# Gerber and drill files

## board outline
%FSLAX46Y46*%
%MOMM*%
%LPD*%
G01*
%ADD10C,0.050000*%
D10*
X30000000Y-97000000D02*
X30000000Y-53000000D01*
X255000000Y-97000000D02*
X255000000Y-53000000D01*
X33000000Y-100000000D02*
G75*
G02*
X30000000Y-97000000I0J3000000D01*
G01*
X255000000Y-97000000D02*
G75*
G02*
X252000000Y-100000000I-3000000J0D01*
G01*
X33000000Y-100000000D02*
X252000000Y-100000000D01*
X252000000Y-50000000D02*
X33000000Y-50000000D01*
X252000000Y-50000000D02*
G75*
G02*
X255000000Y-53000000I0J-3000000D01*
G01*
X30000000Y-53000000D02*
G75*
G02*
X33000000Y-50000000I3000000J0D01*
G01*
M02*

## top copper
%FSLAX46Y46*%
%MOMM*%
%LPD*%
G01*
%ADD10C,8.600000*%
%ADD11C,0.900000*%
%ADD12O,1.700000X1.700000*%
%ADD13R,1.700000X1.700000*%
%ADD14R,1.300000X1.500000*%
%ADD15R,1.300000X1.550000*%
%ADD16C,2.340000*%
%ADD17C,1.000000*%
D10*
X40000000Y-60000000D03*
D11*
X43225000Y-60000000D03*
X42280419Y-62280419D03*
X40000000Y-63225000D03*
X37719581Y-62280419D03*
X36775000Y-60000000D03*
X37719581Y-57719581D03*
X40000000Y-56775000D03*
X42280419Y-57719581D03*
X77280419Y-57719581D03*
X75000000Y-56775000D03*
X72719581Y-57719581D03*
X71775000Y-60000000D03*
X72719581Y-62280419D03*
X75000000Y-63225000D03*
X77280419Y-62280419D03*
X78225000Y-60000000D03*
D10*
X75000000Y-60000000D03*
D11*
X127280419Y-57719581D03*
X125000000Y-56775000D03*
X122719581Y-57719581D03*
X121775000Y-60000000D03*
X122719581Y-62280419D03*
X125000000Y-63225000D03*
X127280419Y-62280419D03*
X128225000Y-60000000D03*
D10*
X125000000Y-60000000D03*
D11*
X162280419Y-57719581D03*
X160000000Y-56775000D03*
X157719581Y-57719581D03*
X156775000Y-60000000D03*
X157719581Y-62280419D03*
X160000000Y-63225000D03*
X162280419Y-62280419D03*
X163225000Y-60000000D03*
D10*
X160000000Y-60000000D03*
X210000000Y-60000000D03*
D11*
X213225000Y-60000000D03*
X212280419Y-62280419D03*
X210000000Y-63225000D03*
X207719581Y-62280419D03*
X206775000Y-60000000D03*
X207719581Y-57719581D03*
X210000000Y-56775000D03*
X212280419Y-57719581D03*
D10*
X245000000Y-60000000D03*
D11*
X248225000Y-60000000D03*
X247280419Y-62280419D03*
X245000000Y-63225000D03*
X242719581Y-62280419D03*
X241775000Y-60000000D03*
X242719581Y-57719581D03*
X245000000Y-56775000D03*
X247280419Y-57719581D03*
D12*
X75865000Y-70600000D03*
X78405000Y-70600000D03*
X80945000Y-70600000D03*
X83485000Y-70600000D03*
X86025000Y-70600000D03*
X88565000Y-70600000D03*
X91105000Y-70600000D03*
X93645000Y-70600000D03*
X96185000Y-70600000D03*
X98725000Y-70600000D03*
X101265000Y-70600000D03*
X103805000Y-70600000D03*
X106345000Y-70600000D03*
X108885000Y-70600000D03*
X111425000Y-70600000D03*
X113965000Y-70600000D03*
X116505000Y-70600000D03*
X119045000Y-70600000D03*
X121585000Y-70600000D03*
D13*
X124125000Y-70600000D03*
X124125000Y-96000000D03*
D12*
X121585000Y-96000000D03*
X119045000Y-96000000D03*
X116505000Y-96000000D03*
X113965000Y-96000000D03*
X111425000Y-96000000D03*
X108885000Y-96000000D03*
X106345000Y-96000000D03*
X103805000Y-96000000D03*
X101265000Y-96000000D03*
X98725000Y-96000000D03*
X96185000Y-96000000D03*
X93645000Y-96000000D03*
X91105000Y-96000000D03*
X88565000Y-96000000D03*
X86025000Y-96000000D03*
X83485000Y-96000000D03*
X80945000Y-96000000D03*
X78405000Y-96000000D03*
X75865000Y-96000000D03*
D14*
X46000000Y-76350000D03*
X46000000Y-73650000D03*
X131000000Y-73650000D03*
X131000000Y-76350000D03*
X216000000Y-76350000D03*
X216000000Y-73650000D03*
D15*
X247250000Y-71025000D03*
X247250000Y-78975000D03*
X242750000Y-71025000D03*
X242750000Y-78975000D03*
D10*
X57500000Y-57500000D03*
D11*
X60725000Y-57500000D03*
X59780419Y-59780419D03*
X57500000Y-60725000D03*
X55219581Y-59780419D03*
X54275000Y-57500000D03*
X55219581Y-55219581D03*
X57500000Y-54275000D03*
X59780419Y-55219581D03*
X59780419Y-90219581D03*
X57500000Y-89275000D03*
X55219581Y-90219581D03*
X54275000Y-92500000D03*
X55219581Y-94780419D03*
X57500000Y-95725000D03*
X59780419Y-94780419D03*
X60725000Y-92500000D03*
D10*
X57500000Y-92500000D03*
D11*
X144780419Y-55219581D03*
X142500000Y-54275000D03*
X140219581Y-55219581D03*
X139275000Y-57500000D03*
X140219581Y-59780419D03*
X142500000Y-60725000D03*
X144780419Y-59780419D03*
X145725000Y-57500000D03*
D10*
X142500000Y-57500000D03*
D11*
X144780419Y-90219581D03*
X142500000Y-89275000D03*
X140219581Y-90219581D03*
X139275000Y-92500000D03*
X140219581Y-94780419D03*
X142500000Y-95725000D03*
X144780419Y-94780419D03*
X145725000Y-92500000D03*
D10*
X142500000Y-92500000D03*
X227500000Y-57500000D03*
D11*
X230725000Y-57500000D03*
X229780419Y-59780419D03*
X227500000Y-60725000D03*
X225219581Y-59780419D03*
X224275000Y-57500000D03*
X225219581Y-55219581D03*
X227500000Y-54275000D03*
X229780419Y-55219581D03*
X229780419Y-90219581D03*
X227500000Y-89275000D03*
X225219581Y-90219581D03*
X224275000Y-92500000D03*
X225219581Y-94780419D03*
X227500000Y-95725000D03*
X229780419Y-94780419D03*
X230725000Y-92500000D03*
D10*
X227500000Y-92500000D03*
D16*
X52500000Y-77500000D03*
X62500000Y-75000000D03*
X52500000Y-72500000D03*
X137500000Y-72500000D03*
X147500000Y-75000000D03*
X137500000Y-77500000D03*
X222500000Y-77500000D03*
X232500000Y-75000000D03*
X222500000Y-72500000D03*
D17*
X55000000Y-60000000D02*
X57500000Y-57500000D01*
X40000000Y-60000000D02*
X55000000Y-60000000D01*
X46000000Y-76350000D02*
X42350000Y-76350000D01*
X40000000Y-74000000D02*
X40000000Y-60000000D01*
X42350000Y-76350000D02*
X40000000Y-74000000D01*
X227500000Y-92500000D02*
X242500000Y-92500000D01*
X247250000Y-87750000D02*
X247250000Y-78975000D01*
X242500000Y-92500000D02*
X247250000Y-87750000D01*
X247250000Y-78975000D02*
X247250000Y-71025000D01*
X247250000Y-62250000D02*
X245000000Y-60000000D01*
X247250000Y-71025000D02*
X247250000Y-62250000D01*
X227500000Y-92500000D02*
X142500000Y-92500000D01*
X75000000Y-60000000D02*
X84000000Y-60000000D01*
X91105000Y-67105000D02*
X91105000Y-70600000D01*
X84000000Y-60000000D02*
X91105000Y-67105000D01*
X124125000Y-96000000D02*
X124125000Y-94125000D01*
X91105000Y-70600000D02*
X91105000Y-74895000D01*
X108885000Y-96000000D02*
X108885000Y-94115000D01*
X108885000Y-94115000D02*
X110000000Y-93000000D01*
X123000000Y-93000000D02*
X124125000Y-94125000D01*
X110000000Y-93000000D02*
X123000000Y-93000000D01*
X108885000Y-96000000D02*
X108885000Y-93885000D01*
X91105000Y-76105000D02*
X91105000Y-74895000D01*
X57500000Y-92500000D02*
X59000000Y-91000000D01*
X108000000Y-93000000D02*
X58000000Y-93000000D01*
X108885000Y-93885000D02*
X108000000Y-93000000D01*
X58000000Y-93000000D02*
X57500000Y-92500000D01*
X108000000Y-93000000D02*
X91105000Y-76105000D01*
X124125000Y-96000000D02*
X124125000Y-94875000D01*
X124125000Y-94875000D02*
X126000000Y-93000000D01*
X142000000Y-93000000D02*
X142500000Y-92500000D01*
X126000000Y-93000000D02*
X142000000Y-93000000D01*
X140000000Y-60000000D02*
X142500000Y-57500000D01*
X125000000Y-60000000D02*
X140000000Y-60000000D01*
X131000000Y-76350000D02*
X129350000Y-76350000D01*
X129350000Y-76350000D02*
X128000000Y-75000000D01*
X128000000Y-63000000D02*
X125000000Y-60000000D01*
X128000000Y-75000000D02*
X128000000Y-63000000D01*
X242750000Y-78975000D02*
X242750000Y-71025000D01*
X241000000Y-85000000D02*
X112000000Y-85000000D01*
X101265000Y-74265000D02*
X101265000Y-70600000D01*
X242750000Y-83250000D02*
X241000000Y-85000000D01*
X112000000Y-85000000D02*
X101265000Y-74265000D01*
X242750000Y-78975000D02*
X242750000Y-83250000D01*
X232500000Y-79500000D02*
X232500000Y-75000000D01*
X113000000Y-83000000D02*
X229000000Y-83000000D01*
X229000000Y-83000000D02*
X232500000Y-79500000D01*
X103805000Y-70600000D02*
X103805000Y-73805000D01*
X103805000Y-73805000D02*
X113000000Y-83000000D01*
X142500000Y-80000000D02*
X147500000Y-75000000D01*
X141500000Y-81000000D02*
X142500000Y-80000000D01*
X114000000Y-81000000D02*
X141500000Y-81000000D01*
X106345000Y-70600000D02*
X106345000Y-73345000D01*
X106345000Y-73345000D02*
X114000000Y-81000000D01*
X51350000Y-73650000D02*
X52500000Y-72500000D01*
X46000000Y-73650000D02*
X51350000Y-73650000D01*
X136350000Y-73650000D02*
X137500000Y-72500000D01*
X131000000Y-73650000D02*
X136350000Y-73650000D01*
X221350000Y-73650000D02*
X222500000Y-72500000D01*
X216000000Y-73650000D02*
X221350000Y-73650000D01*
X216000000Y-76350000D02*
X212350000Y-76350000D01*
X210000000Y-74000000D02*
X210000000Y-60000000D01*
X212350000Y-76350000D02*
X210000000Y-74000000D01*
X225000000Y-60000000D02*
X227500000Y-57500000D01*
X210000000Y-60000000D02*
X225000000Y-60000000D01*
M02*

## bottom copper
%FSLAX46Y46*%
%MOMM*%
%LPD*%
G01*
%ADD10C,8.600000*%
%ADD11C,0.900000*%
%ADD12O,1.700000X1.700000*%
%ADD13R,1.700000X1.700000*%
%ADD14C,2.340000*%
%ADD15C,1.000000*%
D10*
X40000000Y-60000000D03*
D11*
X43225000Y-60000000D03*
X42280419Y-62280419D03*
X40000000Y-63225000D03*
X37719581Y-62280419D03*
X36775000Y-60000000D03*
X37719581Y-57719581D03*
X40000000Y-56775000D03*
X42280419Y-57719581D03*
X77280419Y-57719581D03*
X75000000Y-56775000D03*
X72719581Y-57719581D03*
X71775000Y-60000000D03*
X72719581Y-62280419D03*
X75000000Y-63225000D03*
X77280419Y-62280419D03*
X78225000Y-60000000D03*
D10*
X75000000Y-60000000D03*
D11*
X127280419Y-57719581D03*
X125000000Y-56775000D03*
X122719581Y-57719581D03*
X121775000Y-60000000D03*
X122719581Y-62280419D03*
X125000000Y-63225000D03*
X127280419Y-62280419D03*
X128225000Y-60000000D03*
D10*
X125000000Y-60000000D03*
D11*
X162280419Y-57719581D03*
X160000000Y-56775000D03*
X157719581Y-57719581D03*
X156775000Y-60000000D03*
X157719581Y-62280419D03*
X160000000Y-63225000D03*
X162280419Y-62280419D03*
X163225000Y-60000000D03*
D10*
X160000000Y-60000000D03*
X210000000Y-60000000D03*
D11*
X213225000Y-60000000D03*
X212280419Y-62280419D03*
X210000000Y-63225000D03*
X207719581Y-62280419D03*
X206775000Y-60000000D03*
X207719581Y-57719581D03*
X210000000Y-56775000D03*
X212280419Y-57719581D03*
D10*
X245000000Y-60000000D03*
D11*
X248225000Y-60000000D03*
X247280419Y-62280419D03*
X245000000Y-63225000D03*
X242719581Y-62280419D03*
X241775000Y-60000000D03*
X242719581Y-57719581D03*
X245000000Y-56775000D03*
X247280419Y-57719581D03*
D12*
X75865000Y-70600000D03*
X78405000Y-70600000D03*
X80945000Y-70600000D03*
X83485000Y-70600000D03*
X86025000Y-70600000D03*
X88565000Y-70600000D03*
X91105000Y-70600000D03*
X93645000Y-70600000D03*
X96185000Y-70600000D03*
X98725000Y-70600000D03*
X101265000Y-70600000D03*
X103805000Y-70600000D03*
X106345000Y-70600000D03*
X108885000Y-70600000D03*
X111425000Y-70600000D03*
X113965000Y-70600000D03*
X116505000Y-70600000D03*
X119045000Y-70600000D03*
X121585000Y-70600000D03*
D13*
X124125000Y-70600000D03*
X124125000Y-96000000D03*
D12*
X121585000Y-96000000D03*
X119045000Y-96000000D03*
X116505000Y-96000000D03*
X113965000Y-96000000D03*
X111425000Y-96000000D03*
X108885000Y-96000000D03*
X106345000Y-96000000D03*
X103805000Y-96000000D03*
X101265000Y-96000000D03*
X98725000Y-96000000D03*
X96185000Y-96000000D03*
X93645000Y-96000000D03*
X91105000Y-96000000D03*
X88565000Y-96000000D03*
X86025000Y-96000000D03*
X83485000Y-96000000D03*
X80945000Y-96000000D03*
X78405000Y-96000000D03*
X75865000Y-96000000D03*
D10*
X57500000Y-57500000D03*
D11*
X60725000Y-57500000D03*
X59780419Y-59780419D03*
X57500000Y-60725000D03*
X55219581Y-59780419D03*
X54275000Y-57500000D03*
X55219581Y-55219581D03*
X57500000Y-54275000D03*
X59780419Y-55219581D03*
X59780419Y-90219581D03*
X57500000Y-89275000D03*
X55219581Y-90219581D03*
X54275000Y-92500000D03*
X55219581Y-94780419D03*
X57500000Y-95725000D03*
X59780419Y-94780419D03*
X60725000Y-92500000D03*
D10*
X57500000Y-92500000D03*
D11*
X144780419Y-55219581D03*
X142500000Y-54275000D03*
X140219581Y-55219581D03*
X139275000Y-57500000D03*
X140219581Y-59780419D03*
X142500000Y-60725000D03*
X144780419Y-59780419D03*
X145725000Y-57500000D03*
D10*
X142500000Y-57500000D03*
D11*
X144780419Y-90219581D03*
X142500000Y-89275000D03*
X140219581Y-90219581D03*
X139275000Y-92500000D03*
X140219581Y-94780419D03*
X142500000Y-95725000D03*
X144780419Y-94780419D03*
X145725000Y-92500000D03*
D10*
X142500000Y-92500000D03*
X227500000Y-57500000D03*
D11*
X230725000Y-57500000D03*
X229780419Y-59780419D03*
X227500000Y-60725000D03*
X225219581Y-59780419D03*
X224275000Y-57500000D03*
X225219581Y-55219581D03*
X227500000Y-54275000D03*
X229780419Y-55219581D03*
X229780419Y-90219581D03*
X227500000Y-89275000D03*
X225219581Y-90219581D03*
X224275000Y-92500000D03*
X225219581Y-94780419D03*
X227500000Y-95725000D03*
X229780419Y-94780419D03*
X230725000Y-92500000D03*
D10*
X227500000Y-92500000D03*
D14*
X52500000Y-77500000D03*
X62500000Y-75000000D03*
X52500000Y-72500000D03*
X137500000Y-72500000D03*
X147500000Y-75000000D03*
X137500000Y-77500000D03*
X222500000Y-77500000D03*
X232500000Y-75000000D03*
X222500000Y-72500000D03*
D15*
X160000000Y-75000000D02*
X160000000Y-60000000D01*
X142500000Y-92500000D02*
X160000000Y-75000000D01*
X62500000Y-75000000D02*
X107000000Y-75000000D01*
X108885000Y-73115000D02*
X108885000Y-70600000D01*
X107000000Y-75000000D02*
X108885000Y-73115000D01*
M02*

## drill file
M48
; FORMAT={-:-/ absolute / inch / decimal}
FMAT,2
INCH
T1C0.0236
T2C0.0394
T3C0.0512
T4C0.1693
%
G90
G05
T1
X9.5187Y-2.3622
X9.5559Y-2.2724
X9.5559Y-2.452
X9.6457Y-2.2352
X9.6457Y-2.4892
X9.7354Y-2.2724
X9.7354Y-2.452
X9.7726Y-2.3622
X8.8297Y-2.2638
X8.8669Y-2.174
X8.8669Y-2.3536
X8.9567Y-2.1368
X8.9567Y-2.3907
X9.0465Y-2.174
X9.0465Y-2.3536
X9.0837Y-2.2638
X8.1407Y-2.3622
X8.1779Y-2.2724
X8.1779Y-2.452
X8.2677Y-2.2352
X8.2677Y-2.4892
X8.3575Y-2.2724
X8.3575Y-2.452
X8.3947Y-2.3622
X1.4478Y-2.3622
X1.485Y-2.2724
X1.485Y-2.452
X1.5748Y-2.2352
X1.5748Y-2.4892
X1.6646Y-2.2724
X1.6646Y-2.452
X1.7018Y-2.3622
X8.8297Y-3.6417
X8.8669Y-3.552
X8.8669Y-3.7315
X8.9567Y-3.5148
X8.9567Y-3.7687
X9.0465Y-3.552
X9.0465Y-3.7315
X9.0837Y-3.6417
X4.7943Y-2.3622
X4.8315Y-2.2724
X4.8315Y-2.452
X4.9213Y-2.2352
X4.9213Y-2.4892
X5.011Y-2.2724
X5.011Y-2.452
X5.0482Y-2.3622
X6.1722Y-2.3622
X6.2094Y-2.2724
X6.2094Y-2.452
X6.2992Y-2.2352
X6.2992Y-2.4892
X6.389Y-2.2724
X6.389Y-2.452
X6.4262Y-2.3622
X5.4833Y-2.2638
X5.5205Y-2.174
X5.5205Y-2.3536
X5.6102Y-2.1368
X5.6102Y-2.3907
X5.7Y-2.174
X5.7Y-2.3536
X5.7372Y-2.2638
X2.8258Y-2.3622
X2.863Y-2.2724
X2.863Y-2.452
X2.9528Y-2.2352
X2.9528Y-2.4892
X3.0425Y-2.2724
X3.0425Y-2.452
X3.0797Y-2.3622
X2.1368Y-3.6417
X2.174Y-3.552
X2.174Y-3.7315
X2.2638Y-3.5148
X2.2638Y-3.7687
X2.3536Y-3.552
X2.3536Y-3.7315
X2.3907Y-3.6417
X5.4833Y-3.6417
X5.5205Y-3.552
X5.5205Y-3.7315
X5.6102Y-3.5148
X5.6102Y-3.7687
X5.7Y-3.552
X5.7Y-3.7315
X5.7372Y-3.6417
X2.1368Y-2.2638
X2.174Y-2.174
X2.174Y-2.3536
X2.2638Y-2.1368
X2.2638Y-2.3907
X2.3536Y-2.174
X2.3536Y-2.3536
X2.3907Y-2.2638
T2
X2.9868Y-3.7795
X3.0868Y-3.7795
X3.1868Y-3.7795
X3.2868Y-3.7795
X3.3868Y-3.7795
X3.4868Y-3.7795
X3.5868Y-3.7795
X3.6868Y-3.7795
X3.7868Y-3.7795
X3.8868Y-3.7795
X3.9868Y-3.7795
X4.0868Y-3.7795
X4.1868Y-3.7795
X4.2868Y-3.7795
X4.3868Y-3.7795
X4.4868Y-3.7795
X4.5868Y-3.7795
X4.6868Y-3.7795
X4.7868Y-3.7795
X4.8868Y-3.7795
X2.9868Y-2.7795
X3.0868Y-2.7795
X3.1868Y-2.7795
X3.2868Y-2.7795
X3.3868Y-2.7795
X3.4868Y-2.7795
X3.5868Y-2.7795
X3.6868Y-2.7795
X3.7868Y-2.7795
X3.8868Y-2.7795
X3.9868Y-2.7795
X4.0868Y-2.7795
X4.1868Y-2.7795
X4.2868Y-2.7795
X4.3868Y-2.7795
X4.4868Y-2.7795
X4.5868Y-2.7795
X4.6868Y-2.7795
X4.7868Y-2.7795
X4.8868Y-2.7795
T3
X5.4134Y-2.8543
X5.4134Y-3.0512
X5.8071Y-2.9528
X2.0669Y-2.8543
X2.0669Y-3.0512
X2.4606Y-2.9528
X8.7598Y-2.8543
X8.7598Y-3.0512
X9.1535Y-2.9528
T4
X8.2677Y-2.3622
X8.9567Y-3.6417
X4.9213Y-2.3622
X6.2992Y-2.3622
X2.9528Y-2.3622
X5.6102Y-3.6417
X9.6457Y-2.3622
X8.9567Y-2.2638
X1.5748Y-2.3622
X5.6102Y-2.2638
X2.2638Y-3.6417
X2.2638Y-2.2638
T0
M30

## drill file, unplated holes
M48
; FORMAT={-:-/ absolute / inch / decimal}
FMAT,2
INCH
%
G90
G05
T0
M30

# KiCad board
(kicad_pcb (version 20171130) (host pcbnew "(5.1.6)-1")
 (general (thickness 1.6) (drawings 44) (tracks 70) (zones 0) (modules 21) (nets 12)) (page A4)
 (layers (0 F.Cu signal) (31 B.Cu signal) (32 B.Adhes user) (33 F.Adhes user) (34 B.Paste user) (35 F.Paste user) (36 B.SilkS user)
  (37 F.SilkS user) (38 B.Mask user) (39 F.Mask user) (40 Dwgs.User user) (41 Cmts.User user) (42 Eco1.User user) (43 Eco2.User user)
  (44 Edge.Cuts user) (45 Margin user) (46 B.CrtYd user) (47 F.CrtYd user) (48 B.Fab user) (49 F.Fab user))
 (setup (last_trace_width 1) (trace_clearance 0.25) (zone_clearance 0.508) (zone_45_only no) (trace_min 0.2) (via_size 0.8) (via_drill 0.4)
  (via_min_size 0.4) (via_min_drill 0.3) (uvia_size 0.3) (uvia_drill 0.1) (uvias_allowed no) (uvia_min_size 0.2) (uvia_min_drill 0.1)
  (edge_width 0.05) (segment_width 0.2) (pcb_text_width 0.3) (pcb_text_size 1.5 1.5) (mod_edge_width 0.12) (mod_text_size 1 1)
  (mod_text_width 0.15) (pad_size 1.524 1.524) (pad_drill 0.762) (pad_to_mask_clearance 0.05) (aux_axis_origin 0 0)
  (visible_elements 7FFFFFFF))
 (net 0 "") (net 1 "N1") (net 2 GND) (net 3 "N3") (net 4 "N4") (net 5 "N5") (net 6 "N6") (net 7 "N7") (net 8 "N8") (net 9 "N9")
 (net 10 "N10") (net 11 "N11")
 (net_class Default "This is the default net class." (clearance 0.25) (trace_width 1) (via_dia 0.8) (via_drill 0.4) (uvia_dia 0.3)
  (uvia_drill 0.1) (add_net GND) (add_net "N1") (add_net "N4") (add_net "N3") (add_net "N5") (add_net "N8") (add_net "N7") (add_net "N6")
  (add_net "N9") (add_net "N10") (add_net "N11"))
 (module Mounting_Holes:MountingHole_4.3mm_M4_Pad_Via (layer F.Cu) (at 40 60)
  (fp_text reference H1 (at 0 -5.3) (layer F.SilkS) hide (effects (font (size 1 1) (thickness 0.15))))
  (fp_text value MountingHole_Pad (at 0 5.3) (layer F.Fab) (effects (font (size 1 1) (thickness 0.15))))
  (pad 1 thru_hole circle (at 0 0) (size 8.6 8.6) (drill 4.3) (layers *.Cu *.Mask) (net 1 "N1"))
  (pad 1 thru_hole circle (at 3.225 0) (size 0.9 0.9) (drill 0.6) (layers *.Cu *.Mask) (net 1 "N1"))
  (pad 1 thru_hole circle (at 2.280419 2.280419) (size 0.9 0.9) (drill 0.6) (layers *.Cu *.Mask) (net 1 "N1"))
  (pad 1 thru_hole circle (at 0 3.225) (size 0.9 0.9) (drill 0.6) (layers *.Cu *.Mask) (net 1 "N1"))
  (pad 1 thru_hole circle (at -2.280419 2.280419) (size 0.9 0.9) (drill 0.6) (layers *.Cu *.Mask) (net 1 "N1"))
  (pad 1 thru_hole circle (at -3.225 0) (size 0.9 0.9) (drill 0.6) (layers *.Cu *.Mask) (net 1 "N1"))
  (pad 1 thru_hole circle (at -2.280419 -2.280419) (size 0.9 0.9) (drill 0.6) (layers *.Cu *.Mask) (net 1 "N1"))
  (pad 1 thru_hole circle (at 0 -3.225) (size 0.9 0.9) (drill 0.6) (layers *.Cu *.Mask) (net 1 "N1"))
  (pad 1 thru_hole circle (at 2.280419 -2.280419) (size 0.9 0.9) (drill 0.6) (layers *.Cu *.Mask) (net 1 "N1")))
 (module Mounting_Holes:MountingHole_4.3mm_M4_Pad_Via (layer F.Cu) (at 75 60)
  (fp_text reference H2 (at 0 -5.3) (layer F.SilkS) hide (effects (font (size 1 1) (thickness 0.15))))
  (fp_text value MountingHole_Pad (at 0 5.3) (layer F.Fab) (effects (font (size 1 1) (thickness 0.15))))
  (pad 1 thru_hole circle (at 2.280419 -2.280419) (size 0.9 0.9) (drill 0.6) (layers *.Cu *.Mask) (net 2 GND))
  (pad 1 thru_hole circle (at 0 -3.225) (size 0.9 0.9) (drill 0.6) (layers *.Cu *.Mask) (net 2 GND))
  (pad 1 thru_hole circle (at -2.280419 -2.280419) (size 0.9 0.9) (drill 0.6) (layers *.Cu *.Mask) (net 2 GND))
  (pad 1 thru_hole circle (at -3.225 0) (size 0.9 0.9) (drill 0.6) (layers *.Cu *.Mask) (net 2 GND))
  (pad 1 thru_hole circle (at -2.280419 2.280419) (size 0.9 0.9) (drill 0.6) (layers *.Cu *.Mask) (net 2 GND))
  (pad 1 thru_hole circle (at 0 3.225) (size 0.9 0.9) (drill 0.6) (layers *.Cu *.Mask) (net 2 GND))
  (pad 1 thru_hole circle (at 2.280419 2.280419) (size 0.9 0.9) (drill 0.6) (layers *.Cu *.Mask) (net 2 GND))
  (pad 1 thru_hole circle (at 3.225 0) (size 0.9 0.9) (drill 0.6) (layers *.Cu *.Mask) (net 2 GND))
  (pad 1 thru_hole circle (at 0 0) (size 8.6 8.6) (drill 4.3) (layers *.Cu *.Mask) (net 2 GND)))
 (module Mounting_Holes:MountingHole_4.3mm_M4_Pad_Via (layer F.Cu) (at 125 60)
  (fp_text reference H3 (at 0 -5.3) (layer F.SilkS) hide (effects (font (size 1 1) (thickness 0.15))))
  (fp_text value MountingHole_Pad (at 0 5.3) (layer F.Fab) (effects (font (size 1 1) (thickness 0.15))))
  (pad 1 thru_hole circle (at 2.280419 -2.280419) (size 0.9 0.9) (drill 0.6) (layers *.Cu *.Mask) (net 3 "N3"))
  (pad 1 thru_hole circle (at 0 -3.225) (size 0.9 0.9) (drill 0.6) (layers *.Cu *.Mask) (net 3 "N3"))
  (pad 1 thru_hole circle (at -2.280419 -2.280419) (size 0.9 0.9) (drill 0.6) (layers *.Cu *.Mask) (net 3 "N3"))
  (pad 1 thru_hole circle (at -3.225 0) (size 0.9 0.9) (drill 0.6) (layers *.Cu *.Mask) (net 3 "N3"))
  (pad 1 thru_hole circle (at -2.280419 2.280419) (size 0.9 0.9) (drill 0.6) (layers *.Cu *.Mask) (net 3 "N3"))
  (pad 1 thru_hole circle (at 0 3.225) (size 0.9 0.9) (drill 0.6) (layers *.Cu *.Mask) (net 3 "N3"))
  (pad 1 thru_hole circle (at 2.280419 2.280419) (size 0.9 0.9) (drill 0.6) (layers *.Cu *.Mask) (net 3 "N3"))
  (pad 1 thru_hole circle (at 3.225 0) (size 0.9 0.9) (drill 0.6) (layers *.Cu *.Mask) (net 3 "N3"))
  (pad 1 thru_hole circle (at 0 0) (size 8.6 8.6) (drill 4.3) (layers *.Cu *.Mask) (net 3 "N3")))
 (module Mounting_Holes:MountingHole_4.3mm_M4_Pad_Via (layer F.Cu) (at 160 60)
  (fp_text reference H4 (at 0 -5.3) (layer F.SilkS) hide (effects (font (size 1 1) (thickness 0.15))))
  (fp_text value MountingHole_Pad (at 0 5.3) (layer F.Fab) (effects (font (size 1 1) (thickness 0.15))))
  (pad 1 thru_hole circle (at 2.280419 -2.280419) (size 0.9 0.9) (drill 0.6) (layers *.Cu *.Mask) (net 2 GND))
  (pad 1 thru_hole circle (at 0 -3.225) (size 0.9 0.9) (drill 0.6) (layers *.Cu *.Mask) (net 2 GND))
  (pad 1 thru_hole circle (at -2.280419 -2.280419) (size 0.9 0.9) (drill 0.6) (layers *.Cu *.Mask) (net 2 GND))
  (pad 1 thru_hole circle (at -3.225 0) (size 0.9 0.9) (drill 0.6) (layers *.Cu *.Mask) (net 2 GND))
  (pad 1 thru_hole circle (at -2.280419 2.280419) (size 0.9 0.9) (drill 0.6) (layers *.Cu *.Mask) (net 2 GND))
  (pad 1 thru_hole circle (at 0 3.225) (size 0.9 0.9) (drill 0.6) (layers *.Cu *.Mask) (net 2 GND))
  (pad 1 thru_hole circle (at 2.280419 2.280419) (size 0.9 0.9) (drill 0.6) (layers *.Cu *.Mask) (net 2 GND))
  (pad 1 thru_hole circle (at 3.225 0) (size 0.9 0.9) (drill 0.6) (layers *.Cu *.Mask) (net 2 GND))
  (pad 1 thru_hole circle (at 0 0) (size 8.6 8.6) (drill 4.3) (layers *.Cu *.Mask) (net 2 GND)))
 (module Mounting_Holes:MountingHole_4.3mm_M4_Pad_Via (layer F.Cu) (at 210 60)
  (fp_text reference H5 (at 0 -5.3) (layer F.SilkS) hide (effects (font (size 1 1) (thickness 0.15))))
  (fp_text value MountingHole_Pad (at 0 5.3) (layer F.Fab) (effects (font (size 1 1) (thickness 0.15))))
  (pad 1 thru_hole circle (at 0 0) (size 8.6 8.6) (drill 4.3) (layers *.Cu *.Mask) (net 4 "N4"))
  (pad 1 thru_hole circle (at 3.225 0) (size 0.9 0.9) (drill 0.6) (layers *.Cu *.Mask) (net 4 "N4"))
  (pad 1 thru_hole circle (at 2.280419 2.280419) (size 0.9 0.9) (drill 0.6) (layers *.Cu *.Mask) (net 4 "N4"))
  (pad 1 thru_hole circle (at 0 3.225) (size 0.9 0.9) (drill 0.6) (layers *.Cu *.Mask) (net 4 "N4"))
  (pad 1 thru_hole circle (at -2.280419 2.280419) (size 0.9 0.9) (drill 0.6) (layers *.Cu *.Mask) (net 4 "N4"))
  (pad 1 thru_hole circle (at -3.225 0) (size 0.9 0.9) (drill 0.6) (layers *.Cu *.Mask) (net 4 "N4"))
  (pad 1 thru_hole circle (at -2.280419 -2.280419) (size 0.9 0.9) (drill 0.6) (layers *.Cu *.Mask) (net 4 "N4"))
  (pad 1 thru_hole circle (at 0 -3.225) (size 0.9 0.9) (drill 0.6) (layers *.Cu *.Mask) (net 4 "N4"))
  (pad 1 thru_hole circle (at 2.280419 -2.280419) (size 0.9 0.9) (drill 0.6) (layers *.Cu *.Mask) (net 4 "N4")))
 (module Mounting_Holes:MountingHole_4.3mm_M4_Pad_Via (layer F.Cu) (at 245 60)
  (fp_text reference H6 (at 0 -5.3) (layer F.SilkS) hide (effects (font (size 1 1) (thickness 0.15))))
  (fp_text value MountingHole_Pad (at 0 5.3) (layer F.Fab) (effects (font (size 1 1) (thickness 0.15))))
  (pad 1 thru_hole circle (at 0 0) (size 8.6 8.6) (drill 4.3) (layers *.Cu *.Mask) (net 2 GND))
  (pad 1 thru_hole circle (at 3.225 0) (size 0.9 0.9) (drill 0.6) (layers *.Cu *.Mask) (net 2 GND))
  (pad 1 thru_hole circle (at 2.280419 2.280419) (size 0.9 0.9) (drill 0.6) (layers *.Cu *.Mask) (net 2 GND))
  (pad 1 thru_hole circle (at 0 3.225) (size 0.9 0.9) (drill 0.6) (layers *.Cu *.Mask) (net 2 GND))
  (pad 1 thru_hole circle (at -2.280419 2.280419) (size 0.9 0.9) (drill 0.6) (layers *.Cu *.Mask) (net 2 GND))
  (pad 1 thru_hole circle (at -3.225 0) (size 0.9 0.9) (drill 0.6) (layers *.Cu *.Mask) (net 2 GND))
  (pad 1 thru_hole circle (at -2.280419 -2.280419) (size 0.9 0.9) (drill 0.6) (layers *.Cu *.Mask) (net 2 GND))
  (pad 1 thru_hole circle (at 0 -3.225) (size 0.9 0.9) (drill 0.6) (layers *.Cu *.Mask) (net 2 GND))
  (pad 1 thru_hole circle (at 2.280419 -2.280419) (size 0.9 0.9) (drill 0.6) (layers *.Cu *.Mask) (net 2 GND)))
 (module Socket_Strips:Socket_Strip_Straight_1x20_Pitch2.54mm (layer F.Cu) (at 124.125 70.6 270)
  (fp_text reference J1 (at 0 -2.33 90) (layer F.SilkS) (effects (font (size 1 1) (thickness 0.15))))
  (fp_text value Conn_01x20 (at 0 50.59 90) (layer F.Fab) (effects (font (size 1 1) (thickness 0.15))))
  (pad 20 thru_hole oval (at 0 48.26 270) (size 1.7 1.7) (drill 1) (layers *.Cu *.Mask))
  (pad 19 thru_hole oval (at 0 45.72 270) (size 1.7 1.7) (drill 1) (layers *.Cu *.Mask))
  (pad 18 thru_hole oval (at 0 43.18 270) (size 1.7 1.7) (drill 1) (layers *.Cu *.Mask))
  (pad 17 thru_hole oval (at 0 40.64 270) (size 1.7 1.7) (drill 1) (layers *.Cu *.Mask))
  (pad 16 thru_hole oval (at 0 38.1 270) (size 1.7 1.7) (drill 1) (layers *.Cu *.Mask))
  (pad 15 thru_hole oval (at 0 35.56 270) (size 1.7 1.7) (drill 1) (layers *.Cu *.Mask))
  (pad 14 thru_hole oval (at 0 33.02 270) (size 1.7 1.7) (drill 1) (layers *.Cu *.Mask) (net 2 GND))
  (pad 13 thru_hole oval (at 0 30.48 270) (size 1.7 1.7) (drill 1) (layers *.Cu *.Mask))
  (pad 12 thru_hole oval (at 0 27.94 270) (size 1.7 1.7) (drill 1) (layers *.Cu *.Mask))
  (pad 11 thru_hole oval (at 0 25.4 270) (size 1.7 1.7) (drill 1) (layers *.Cu *.Mask))
  (pad 10 thru_hole oval (at 0 22.86 270) (size 1.7 1.7) (drill 1) (layers *.Cu *.Mask) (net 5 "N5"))
  (pad 9 thru_hole oval (at 0 20.32 270) (size 1.7 1.7) (drill 1) (layers *.Cu *.Mask) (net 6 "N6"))
  (pad 8 thru_hole oval (at 0 17.78 270) (size 1.7 1.7) (drill 1) (layers *.Cu *.Mask) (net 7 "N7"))
  (pad 7 thru_hole oval (at 0 15.24 270) (size 1.7 1.7) (drill 1) (layers *.Cu *.Mask) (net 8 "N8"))
  (pad 6 thru_hole oval (at 0 12.7 270) (size 1.7 1.7) (drill 1) (layers *.Cu *.Mask))
  (pad 5 thru_hole oval (at 0 10.16 270) (size 1.7 1.7) (drill 1) (layers *.Cu *.Mask))
  (pad 4 thru_hole oval (at 0 7.62 270) (size 1.7 1.7) (drill 1) (layers *.Cu *.Mask))
  (pad 3 thru_hole oval (at 0 5.08 270) (size 1.7 1.7) (drill 1) (layers *.Cu *.Mask))
  (pad 2 thru_hole oval (at 0 2.54 270) (size 1.7 1.7) (drill 1) (layers *.Cu *.Mask))
  (pad 1 thru_hole rect (at 0 0 270) (size 1.7 1.7) (drill 1) (layers *.Cu *.Mask)))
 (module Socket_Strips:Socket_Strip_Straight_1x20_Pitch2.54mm (layer F.Cu) (at 124.125 96 270)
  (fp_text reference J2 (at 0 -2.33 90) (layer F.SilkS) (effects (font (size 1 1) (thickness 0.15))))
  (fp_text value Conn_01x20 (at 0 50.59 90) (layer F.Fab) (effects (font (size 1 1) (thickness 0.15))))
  (pad 1 thru_hole rect (at 0 0 270) (size 1.7 1.7) (drill 1) (layers *.Cu *.Mask) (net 2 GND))
  (pad 2 thru_hole oval (at 0 2.54 270) (size 1.7 1.7) (drill 1) (layers *.Cu *.Mask))
  (pad 3 thru_hole oval (at 0 5.08 270) (size 1.7 1.7) (drill 1) (layers *.Cu *.Mask))
  (pad 4 thru_hole oval (at 0 7.62 270) (size 1.7 1.7) (drill 1) (layers *.Cu *.Mask))
  (pad 5 thru_hole oval (at 0 10.16 270) (size 1.7 1.7) (drill 1) (layers *.Cu *.Mask))
  (pad 6 thru_hole oval (at 0 12.7 270) (size 1.7 1.7) (drill 1) (layers *.Cu *.Mask))
  (pad 7 thru_hole oval (at 0 15.24 270) (size 1.7 1.7) (drill 1) (layers *.Cu *.Mask) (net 2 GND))
  (pad 8 thru_hole oval (at 0 17.78 270) (size 1.7 1.7) (drill 1) (layers *.Cu *.Mask))
  (pad 9 thru_hole oval (at 0 20.32 270) (size 1.7 1.7) (drill 1) (layers *.Cu *.Mask))
  (pad 10 thru_hole oval (at 0 22.86 270) (size 1.7 1.7) (drill 1) (layers *.Cu *.Mask))
  (pad 11 thru_hole oval (at 0 25.4 270) (size 1.7 1.7) (drill 1) (layers *.Cu *.Mask))
  (pad 12 thru_hole oval (at 0 27.94 270) (size 1.7 1.7) (drill 1) (layers *.Cu *.Mask))
  (pad 13 thru_hole oval (at 0 30.48 270) (size 1.7 1.7) (drill 1) (layers *.Cu *.Mask))
  (pad 14 thru_hole oval (at 0 33.02 270) (size 1.7 1.7) (drill 1) (layers *.Cu *.Mask))
  (pad 15 thru_hole oval (at 0 35.56 270) (size 1.7 1.7) (drill 1) (layers *.Cu *.Mask))
  (pad 16 thru_hole oval (at 0 38.1 270) (size 1.7 1.7) (drill 1) (layers *.Cu *.Mask))
  (pad 17 thru_hole oval (at 0 40.64 270) (size 1.7 1.7) (drill 1) (layers *.Cu *.Mask))
  (pad 18 thru_hole oval (at 0 43.18 270) (size 1.7 1.7) (drill 1) (layers *.Cu *.Mask))
  (pad 19 thru_hole oval (at 0 45.72 270) (size 1.7 1.7) (drill 1) (layers *.Cu *.Mask))
  (pad 20 thru_hole oval (at 0 48.26 270) (size 1.7 1.7) (drill 1) (layers *.Cu *.Mask)))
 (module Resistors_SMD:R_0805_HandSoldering (layer F.Cu) (at 46 75 270)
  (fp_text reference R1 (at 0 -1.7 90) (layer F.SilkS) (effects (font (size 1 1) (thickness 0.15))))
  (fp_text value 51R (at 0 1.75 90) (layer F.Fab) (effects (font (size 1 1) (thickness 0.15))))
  (pad 2 smd rect (at 1.35 0 270) (size 1.5 1.3) (layers F.Cu F.Paste F.Mask) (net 1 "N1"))
  (pad 1 smd rect (at -1.35 0 270) (size 1.5 1.3) (layers F.Cu F.Paste F.Mask) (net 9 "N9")))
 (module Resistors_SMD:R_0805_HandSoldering (layer F.Cu) (at 131 75 270)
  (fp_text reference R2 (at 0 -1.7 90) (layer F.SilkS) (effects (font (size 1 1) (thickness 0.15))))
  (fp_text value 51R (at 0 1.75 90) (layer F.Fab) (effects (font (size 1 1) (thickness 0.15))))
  (pad 1 smd rect (at -1.35 0 270) (size 1.5 1.3) (layers F.Cu F.Paste F.Mask) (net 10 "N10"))
  (pad 2 smd rect (at 1.35 0 270) (size 1.5 1.3) (layers F.Cu F.Paste F.Mask) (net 3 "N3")))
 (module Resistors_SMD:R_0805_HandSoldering (layer F.Cu) (at 216 75 270)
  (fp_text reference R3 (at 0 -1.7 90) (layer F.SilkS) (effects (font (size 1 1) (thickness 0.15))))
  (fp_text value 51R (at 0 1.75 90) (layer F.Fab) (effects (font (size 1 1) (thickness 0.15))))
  (pad 2 smd rect (at 1.35 0 270) (size 1.5 1.3) (layers F.Cu F.Paste F.Mask) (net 4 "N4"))
  (pad 1 smd rect (at -1.35 0 270) (size 1.5 1.3) (layers F.Cu F.Paste F.Mask) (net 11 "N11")))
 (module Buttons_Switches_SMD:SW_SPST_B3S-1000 (layer F.Cu) (at 245 75 90)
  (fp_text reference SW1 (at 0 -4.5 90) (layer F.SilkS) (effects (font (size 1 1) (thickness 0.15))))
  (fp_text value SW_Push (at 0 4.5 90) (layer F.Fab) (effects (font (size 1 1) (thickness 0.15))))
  (pad 2 smd rect (at 3.975 2.25 90) (size 1.55 1.3) (layers F.Cu F.Paste F.Mask) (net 2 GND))
  (pad 2 smd rect (at -3.975 2.25 90) (size 1.55 1.3) (layers F.Cu F.Paste F.Mask) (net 2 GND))
  (pad 1 smd rect (at 3.975 -2.25 90) (size 1.55 1.3) (layers F.Cu F.Paste F.Mask) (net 5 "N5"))
  (pad 1 smd rect (at -3.975 -2.25 90) (size 1.55 1.3) (layers F.Cu F.Paste F.Mask) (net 5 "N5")))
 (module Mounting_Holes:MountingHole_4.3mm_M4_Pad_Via (layer F.Cu) (at 57.5 57.5)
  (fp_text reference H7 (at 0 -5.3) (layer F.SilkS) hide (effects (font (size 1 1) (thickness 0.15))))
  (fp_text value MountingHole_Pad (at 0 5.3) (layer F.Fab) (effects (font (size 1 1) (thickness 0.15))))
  (pad 1 thru_hole circle (at 0 0) (size 8.6 8.6) (drill 4.3) (layers *.Cu *.Mask) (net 1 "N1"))
  (pad 1 thru_hole circle (at 3.225 0) (size 0.9 0.9) (drill 0.6) (layers *.Cu *.Mask) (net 1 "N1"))
  (pad 1 thru_hole circle (at 2.280419 2.280419) (size 0.9 0.9) (drill 0.6) (layers *.Cu *.Mask) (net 1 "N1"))
  (pad 1 thru_hole circle (at 0 3.225) (size 0.9 0.9) (drill 0.6) (layers *.Cu *.Mask) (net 1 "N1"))
  (pad 1 thru_hole circle (at -2.280419 2.280419) (size 0.9 0.9) (drill 0.6) (layers *.Cu *.Mask) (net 1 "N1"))
  (pad 1 thru_hole circle (at -3.225 0) (size 0.9 0.9) (drill 0.6) (layers *.Cu *.Mask) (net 1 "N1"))
  (pad 1 thru_hole circle (at -2.280419 -2.280419) (size 0.9 0.9) (drill 0.6) (layers *.Cu *.Mask) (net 1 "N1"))
  (pad 1 thru_hole circle (at 0 -3.225) (size 0.9 0.9) (drill 0.6) (layers *.Cu *.Mask) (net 1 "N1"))
  (pad 1 thru_hole circle (at 2.280419 -2.280419) (size 0.9 0.9) (drill 0.6) (layers *.Cu *.Mask) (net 1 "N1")))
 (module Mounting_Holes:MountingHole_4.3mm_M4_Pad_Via (layer F.Cu) (at 57.5 92.5)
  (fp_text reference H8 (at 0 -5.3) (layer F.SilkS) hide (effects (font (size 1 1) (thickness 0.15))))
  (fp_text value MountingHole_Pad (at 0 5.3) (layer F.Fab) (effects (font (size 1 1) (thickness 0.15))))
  (pad 1 thru_hole circle (at 2.280419 -2.280419) (size 0.9 0.9) (drill 0.6) (layers *.Cu *.Mask) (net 2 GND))
  (pad 1 thru_hole circle (at 0 -3.225) (size 0.9 0.9) (drill 0.6) (layers *.Cu *.Mask) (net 2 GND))
  (pad 1 thru_hole circle (at -2.280419 -2.280419) (size 0.9 0.9) (drill 0.6) (layers *.Cu *.Mask) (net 2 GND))
  (pad 1 thru_hole circle (at -3.225 0) (size 0.9 0.9) (drill 0.6) (layers *.Cu *.Mask) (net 2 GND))
  (pad 1 thru_hole circle (at -2.280419 2.280419) (size 0.9 0.9) (drill 0.6) (layers *.Cu *.Mask) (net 2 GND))
  (pad 1 thru_hole circle (at 0 3.225) (size 0.9 0.9) (drill 0.6) (layers *.Cu *.Mask) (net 2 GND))
  (pad 1 thru_hole circle (at 2.280419 2.280419) (size 0.9 0.9) (drill 0.6) (layers *.Cu *.Mask) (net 2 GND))
  (pad 1 thru_hole circle (at 3.225 0) (size 0.9 0.9) (drill 0.6) (layers *.Cu *.Mask) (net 2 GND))
  (pad 1 thru_hole circle (at 0 0) (size 8.6 8.6) (drill 4.3) (layers *.Cu *.Mask) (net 2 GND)))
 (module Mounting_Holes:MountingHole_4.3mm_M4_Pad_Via (layer F.Cu) (at 142.5 57.5)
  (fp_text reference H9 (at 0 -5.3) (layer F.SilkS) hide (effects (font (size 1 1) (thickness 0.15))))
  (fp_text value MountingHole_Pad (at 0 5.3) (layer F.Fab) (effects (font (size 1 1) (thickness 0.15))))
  (pad 1 thru_hole circle (at 2.280419 -2.280419) (size 0.9 0.9) (drill 0.6) (layers *.Cu *.Mask) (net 3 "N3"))
  (pad 1 thru_hole circle (at 0 -3.225) (size 0.9 0.9) (drill 0.6) (layers *.Cu *.Mask) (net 3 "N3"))
  (pad 1 thru_hole circle (at -2.280419 -2.280419) (size 0.9 0.9) (drill 0.6) (layers *.Cu *.Mask) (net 3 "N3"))
  (pad 1 thru_hole circle (at -3.225 0) (size 0.9 0.9) (drill 0.6) (layers *.Cu *.Mask) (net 3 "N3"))
  (pad 1 thru_hole circle (at -2.280419 2.280419) (size 0.9 0.9) (drill 0.6) (layers *.Cu *.Mask) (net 3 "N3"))
  (pad 1 thru_hole circle (at 0 3.225) (size 0.9 0.9) (drill 0.6) (layers *.Cu *.Mask) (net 3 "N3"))
  (pad 1 thru_hole circle (at 2.280419 2.280419) (size 0.9 0.9) (drill 0.6) (layers *.Cu *.Mask) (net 3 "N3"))
  (pad 1 thru_hole circle (at 3.225 0) (size 0.9 0.9) (drill 0.6) (layers *.Cu *.Mask) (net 3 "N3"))
  (pad 1 thru_hole circle (at 0 0) (size 8.6 8.6) (drill 4.3) (layers *.Cu *.Mask) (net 3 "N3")))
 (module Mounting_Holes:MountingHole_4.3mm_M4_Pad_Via (layer F.Cu) (at 142.5 92.5)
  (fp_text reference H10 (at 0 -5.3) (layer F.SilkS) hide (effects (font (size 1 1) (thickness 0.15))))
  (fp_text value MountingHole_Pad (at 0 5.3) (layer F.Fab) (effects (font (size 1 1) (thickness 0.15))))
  (pad 1 thru_hole circle (at 2.280419 -2.280419) (size 0.9 0.9) (drill 0.6) (layers *.Cu *.Mask) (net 2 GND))
  (pad 1 thru_hole circle (at 0 -3.225) (size 0.9 0.9) (drill 0.6) (layers *.Cu *.Mask) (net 2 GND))
  (pad 1 thru_hole circle (at -2.280419 -2.280419) (size 0.9 0.9) (drill 0.6) (layers *.Cu *.Mask) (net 2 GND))
  (pad 1 thru_hole circle (at -3.225 0) (size 0.9 0.9) (drill 0.6) (layers *.Cu *.Mask) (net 2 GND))
  (pad 1 thru_hole circle (at -2.280419 2.280419) (size 0.9 0.9) (drill 0.6) (layers *.Cu *.Mask) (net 2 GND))
  (pad 1 thru_hole circle (at 0 3.225) (size 0.9 0.9) (drill 0.6) (layers *.Cu *.Mask) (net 2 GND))
  (pad 1 thru_hole circle (at 2.280419 2.280419) (size 0.9 0.9) (drill 0.6) (layers *.Cu *.Mask) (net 2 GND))
  (pad 1 thru_hole circle (at 3.225 0) (size 0.9 0.9) (drill 0.6) (layers *.Cu *.Mask) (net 2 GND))
  (pad 1 thru_hole circle (at 0 0) (size 8.6 8.6) (drill 4.3) (layers *.Cu *.Mask) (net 2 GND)))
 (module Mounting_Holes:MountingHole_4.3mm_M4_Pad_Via (layer F.Cu) (at 227.5 57.5)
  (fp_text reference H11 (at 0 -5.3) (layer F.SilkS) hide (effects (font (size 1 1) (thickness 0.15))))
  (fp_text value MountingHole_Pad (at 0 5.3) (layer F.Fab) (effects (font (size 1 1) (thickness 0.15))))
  (pad 1 thru_hole circle (at 0 0) (size 8.6 8.6) (drill 4.3) (layers *.Cu *.Mask) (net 4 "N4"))
  (pad 1 thru_hole circle (at 3.225 0) (size 0.9 0.9) (drill 0.6) (layers *.Cu *.Mask) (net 4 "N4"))
  (pad 1 thru_hole circle (at 2.280419 2.280419) (size 0.9 0.9) (drill 0.6) (layers *.Cu *.Mask) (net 4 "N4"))
  (pad 1 thru_hole circle (at 0 3.225) (size 0.9 0.9) (drill 0.6) (layers *.Cu *.Mask) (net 4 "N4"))
  (pad 1 thru_hole circle (at -2.280419 2.280419) (size 0.9 0.9) (drill 0.6) (layers *.Cu *.Mask) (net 4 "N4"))
  (pad 1 thru_hole circle (at -3.225 0) (size 0.9 0.9) (drill 0.6) (layers *.Cu *.Mask) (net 4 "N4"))
  (pad 1 thru_hole circle (at -2.280419 -2.280419) (size 0.9 0.9) (drill 0.6) (layers *.Cu *.Mask) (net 4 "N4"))
  (pad 1 thru_hole circle (at 0 -3.225) (size 0.9 0.9) (drill 0.6) (layers *.Cu *.Mask) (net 4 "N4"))
  (pad 1 thru_hole circle (at 2.280419 -2.280419) (size 0.9 0.9) (drill 0.6) (layers *.Cu *.Mask) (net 4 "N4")))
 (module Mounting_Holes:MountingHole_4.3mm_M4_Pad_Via (layer F.Cu) (at 227.5 92.5)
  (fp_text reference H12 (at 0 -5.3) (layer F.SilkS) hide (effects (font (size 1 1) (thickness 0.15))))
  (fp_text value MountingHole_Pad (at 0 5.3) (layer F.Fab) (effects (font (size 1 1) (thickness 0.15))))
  (pad 1 thru_hole circle (at 2.280419 -2.280419) (size 0.9 0.9) (drill 0.6) (layers *.Cu *.Mask) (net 2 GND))
  (pad 1 thru_hole circle (at 0 -3.225) (size 0.9 0.9) (drill 0.6) (layers *.Cu *.Mask) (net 2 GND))
  (pad 1 thru_hole circle (at -2.280419 -2.280419) (size 0.9 0.9) (drill 0.6) (layers *.Cu *.Mask) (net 2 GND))
  (pad 1 thru_hole circle (at -3.225 0) (size 0.9 0.9) (drill 0.6) (layers *.Cu *.Mask) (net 2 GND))
  (pad 1 thru_hole circle (at -2.280419 2.280419) (size 0.9 0.9) (drill 0.6) (layers *.Cu *.Mask) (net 2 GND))
  (pad 1 thru_hole circle (at 0 3.225) (size 0.9 0.9) (drill 0.6) (layers *.Cu *.Mask) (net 2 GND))
  (pad 1 thru_hole circle (at 2.280419 2.280419) (size 0.9 0.9) (drill 0.6) (layers *.Cu *.Mask) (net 2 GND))
  (pad 1 thru_hole circle (at 3.225 0) (size 0.9 0.9) (drill 0.6) (layers *.Cu *.Mask) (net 2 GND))
  (pad 1 thru_hole circle (at 0 0) (size 8.6 8.6) (drill 4.3) (layers *.Cu *.Mask) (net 2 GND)))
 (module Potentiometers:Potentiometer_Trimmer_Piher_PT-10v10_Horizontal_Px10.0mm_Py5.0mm (layer F.Cu) (at 52.5 77.5)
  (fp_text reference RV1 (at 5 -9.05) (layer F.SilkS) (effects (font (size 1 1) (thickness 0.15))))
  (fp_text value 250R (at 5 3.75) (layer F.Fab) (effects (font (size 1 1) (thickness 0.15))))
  (pad 1 thru_hole circle (at 0 0) (size 2.34 2.34) (drill 1.3) (layers *.Cu *.Mask))
  (pad 2 thru_hole circle (at 10 -2.5) (size 2.34 2.34) (drill 1.3) (layers *.Cu *.Mask) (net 8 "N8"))
  (pad 3 thru_hole circle (at 0 -5) (size 2.34 2.34) (drill 1.3) (layers *.Cu *.Mask) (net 9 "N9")))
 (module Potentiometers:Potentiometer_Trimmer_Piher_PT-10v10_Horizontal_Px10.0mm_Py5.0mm (layer F.Cu) (at 137.5 77.5)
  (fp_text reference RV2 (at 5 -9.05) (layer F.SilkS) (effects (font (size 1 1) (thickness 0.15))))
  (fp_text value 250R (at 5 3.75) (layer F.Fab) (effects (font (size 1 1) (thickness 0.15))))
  (pad 3 thru_hole circle (at 0 -5) (size 2.34 2.34) (drill 1.3) (layers *.Cu *.Mask) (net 10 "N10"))
  (pad 2 thru_hole circle (at 10 -2.5) (size 2.34 2.34) (drill 1.3) (layers *.Cu *.Mask) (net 7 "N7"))
  (pad 1 thru_hole circle (at 0 0) (size 2.34 2.34) (drill 1.3) (layers *.Cu *.Mask)))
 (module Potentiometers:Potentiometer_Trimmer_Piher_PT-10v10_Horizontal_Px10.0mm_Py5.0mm (layer F.Cu) (at 222.5 77.5)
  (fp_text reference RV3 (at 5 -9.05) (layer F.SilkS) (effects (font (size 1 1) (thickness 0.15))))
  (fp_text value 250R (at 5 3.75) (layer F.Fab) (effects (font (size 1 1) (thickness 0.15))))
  (pad 1 thru_hole circle (at 0 0) (size 2.34 2.34) (drill 1.3) (layers *.Cu *.Mask))
  (pad 2 thru_hole circle (at 10 -2.5) (size 2.34 2.34) (drill 1.3) (layers *.Cu *.Mask) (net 6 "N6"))
  (pad 3 thru_hole circle (at 0 -5) (size 2.34 2.34) (drill 1.3) (layers *.Cu *.Mask) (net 11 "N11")))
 (gr_line (start 30 97) (end 30 53) (layer Edge.Cuts) (width 0.05))
 (gr_line (start 255 97) (end 255 53) (layer Edge.Cuts) (width 0.05))
 (gr_arc (start 33 97) (end 30 97) (angle -90) (layer Edge.Cuts) (width 0.05))
 (gr_arc (start 252 97) (end 252 100) (angle -90) (layer Edge.Cuts) (width 0.05))
 (gr_line (start 33 100) (end 252 100) (layer Edge.Cuts) (width 0.05))
 (gr_line (start 252 50) (end 33 50) (layer Edge.Cuts) (width 0.05))
 (gr_arc (start 252 53) (end 255 53) (angle -90) (layer Edge.Cuts) (width 0.05))
 (gr_arc (start 33 53) (end 33 50) (angle -90) (layer Edge.Cuts) (width 0.05))
 (segment (start 55 60) (end 57.5 57.5) (width 1) (layer F.Cu) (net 1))
 (segment (start 40 60) (end 55 60) (width 1) (layer F.Cu) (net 1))
 (segment (start 46 76.35) (end 42.35 76.35) (width 1) (layer F.Cu) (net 1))
 (segment (start 40 74) (end 40 60) (width 1) (layer F.Cu) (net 1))
 (segment (start 42.35 76.35) (end 40 74) (width 1) (layer F.Cu) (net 1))
 (segment (start 227.5 92.5) (end 242.5 92.5) (width 1) (layer F.Cu) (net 2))
 (segment (start 247.25 87.75) (end 247.25 78.975) (width 1) (layer F.Cu) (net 2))
 (segment (start 242.5 92.5) (end 247.25 87.75) (width 1) (layer F.Cu) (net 2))
 (segment (start 247.25 78.975) (end 247.25 71.025) (width 1) (layer F.Cu) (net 2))
 (segment (start 247.25 62.25) (end 245 60) (width 1) (layer F.Cu) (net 2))
 (segment (start 247.25 71.025) (end 247.25 62.25) (width 1) (layer F.Cu) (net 2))
 (segment (start 227.5 92.5) (end 142.5 92.5) (width 1) (layer F.Cu) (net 2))
 (segment (start 75 60) (end 84 60) (width 1) (layer F.Cu) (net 2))
 (segment (start 91.105 67.105) (end 91.105 70.6) (width 1) (layer F.Cu) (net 2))
 (segment (start 84 60) (end 91.105 67.105) (width 1) (layer F.Cu) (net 2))
 (segment (start 160 75) (end 160 60) (width 1) (layer B.Cu) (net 2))
 (segment (start 142.5 92.5) (end 160 75) (width 1) (layer B.Cu) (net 2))
 (segment (start 124.125 96) (end 124.125 94.125) (width 1) (layer F.Cu) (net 2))
 (segment (start 91.105 70.6) (end 91.105 74.895) (width 1) (layer F.Cu) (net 2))
 (segment (start 108.885 96) (end 108.885 94.115) (width 1) (layer F.Cu) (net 2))
 (segment (start 108.885 94.115) (end 110 93) (width 1) (layer F.Cu) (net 2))
 (segment (start 123 93) (end 124.125 94.125) (width 1) (layer F.Cu) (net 2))
 (segment (start 110 93) (end 123 93) (width 1) (layer F.Cu) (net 2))
 (segment (start 108.885 96) (end 108.885 93.885) (width 1) (layer F.Cu) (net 2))
 (segment (start 91.105 76.105) (end 91.105 74.895) (width 1) (layer F.Cu) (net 2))
 (segment (start 57.5 92.5) (end 59 91) (width 1) (layer F.Cu) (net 2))
 (segment (start 108 93) (end 58 93) (width 1) (layer F.Cu) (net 2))
 (segment (start 108.885 93.885) (end 108 93) (width 1) (layer F.Cu) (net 2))
 (segment (start 58 93) (end 57.5 92.5) (width 1) (layer F.Cu) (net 2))
 (segment (start 108 93) (end 91.105 76.105) (width 1) (layer F.Cu) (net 2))
 (segment (start 124.125 96) (end 124.125 94.875) (width 1) (layer F.Cu) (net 2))
 (segment (start 124.125 94.875) (end 126 93) (width 1) (layer F.Cu) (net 2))
 (segment (start 142 93) (end 142.5 92.5) (width 1) (layer F.Cu) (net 2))
 (segment (start 126 93) (end 142 93) (width 1) (layer F.Cu) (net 2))
 (segment (start 140 60) (end 142.5 57.5) (width 1) (layer F.Cu) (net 3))
 (segment (start 125 60) (end 140 60) (width 1) (layer F.Cu) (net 3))
 (segment (start 131 76.35) (end 129.35 76.35) (width 1) (layer F.Cu) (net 3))
 (segment (start 129.35 76.35) (end 128 75) (width 1) (layer F.Cu) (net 3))
 (segment (start 128 63) (end 125 60) (width 1) (layer F.Cu) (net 3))
 (segment (start 128 75) (end 128 63) (width 1) (layer F.Cu) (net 3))
 (segment (start 242.75 78.975) (end 242.75 71.025) (width 1) (layer F.Cu) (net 5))
 (segment (start 241 85) (end 112 85) (width 1) (layer F.Cu) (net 5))
 (segment (start 101.265 74.265) (end 101.265 70.6) (width 1) (layer F.Cu) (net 5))
 (segment (start 242.75 83.25) (end 241 85) (width 1) (layer F.Cu) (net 5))
 (segment (start 112 85) (end 101.265 74.265) (width 1) (layer F.Cu) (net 5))
 (segment (start 242.75 78.975) (end 242.75 83.25) (width 1) (layer F.Cu) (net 5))
 (segment (start 232.5 79.5) (end 232.5 75) (width 1) (layer F.Cu) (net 6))
 (segment (start 113 83) (end 229 83) (width 1) (layer F.Cu) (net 6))
 (segment (start 229 83) (end 232.5 79.5) (width 1) (layer F.Cu) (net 6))
 (segment (start 103.805 70.6) (end 103.805 73.805) (width 1) (layer F.Cu) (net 6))
 (segment (start 103.805 73.805) (end 113 83) (width 1) (layer F.Cu) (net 6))
 (segment (start 142.5 80) (end 147.5 75) (width 1) (layer F.Cu) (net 7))
 (segment (start 141.5 81) (end 142.5 80) (width 1) (layer F.Cu) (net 7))
 (segment (start 114 81) (end 141.5 81) (width 1) (layer F.Cu) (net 7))
 (segment (start 106.345 70.6) (end 106.345 73.345) (width 1) (layer F.Cu) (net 7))
 (segment (start 106.345 73.345) (end 114 81) (width 1) (layer F.Cu) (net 7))
 (segment (start 62.5 75) (end 107 75) (width 1) (layer B.Cu) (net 8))
 (segment (start 108.885 73.115) (end 108.885 70.6) (width 1) (layer B.Cu) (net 8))
 (segment (start 107 75) (end 108.885 73.115) (width 1) (layer B.Cu) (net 8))
 (segment (start 51.35 73.65) (end 52.5 72.5) (width 1) (layer F.Cu) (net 9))
 (segment (start 46 73.65) (end 51.35 73.65) (width 1) (layer F.Cu) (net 9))
 (segment (start 136.35 73.65) (end 137.5 72.5) (width 1) (layer F.Cu) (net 10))
 (segment (start 131 73.65) (end 136.35 73.65) (width 1) (layer F.Cu) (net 10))
 (segment (start 221.35 73.65) (end 222.5 72.5) (width 1) (layer F.Cu) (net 11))
 (segment (start 216 73.65) (end 221.35 73.65) (width 1) (layer F.Cu) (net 11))
 (segment (start 216 76.35) (end 212.35 76.35) (width 1) (layer F.Cu) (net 4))
 (segment (start 210 74) (end 210 60) (width 1) (layer F.Cu) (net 4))
 (segment (start 212.35 76.35) (end 210 74) (width 1) (layer F.Cu) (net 4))
 (segment (start 225 60) (end 227.5 57.5) (width 1) (layer F.Cu) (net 4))
 (segment (start 210 60) (end 225 60) (width 1) (layer F.Cu) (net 4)))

